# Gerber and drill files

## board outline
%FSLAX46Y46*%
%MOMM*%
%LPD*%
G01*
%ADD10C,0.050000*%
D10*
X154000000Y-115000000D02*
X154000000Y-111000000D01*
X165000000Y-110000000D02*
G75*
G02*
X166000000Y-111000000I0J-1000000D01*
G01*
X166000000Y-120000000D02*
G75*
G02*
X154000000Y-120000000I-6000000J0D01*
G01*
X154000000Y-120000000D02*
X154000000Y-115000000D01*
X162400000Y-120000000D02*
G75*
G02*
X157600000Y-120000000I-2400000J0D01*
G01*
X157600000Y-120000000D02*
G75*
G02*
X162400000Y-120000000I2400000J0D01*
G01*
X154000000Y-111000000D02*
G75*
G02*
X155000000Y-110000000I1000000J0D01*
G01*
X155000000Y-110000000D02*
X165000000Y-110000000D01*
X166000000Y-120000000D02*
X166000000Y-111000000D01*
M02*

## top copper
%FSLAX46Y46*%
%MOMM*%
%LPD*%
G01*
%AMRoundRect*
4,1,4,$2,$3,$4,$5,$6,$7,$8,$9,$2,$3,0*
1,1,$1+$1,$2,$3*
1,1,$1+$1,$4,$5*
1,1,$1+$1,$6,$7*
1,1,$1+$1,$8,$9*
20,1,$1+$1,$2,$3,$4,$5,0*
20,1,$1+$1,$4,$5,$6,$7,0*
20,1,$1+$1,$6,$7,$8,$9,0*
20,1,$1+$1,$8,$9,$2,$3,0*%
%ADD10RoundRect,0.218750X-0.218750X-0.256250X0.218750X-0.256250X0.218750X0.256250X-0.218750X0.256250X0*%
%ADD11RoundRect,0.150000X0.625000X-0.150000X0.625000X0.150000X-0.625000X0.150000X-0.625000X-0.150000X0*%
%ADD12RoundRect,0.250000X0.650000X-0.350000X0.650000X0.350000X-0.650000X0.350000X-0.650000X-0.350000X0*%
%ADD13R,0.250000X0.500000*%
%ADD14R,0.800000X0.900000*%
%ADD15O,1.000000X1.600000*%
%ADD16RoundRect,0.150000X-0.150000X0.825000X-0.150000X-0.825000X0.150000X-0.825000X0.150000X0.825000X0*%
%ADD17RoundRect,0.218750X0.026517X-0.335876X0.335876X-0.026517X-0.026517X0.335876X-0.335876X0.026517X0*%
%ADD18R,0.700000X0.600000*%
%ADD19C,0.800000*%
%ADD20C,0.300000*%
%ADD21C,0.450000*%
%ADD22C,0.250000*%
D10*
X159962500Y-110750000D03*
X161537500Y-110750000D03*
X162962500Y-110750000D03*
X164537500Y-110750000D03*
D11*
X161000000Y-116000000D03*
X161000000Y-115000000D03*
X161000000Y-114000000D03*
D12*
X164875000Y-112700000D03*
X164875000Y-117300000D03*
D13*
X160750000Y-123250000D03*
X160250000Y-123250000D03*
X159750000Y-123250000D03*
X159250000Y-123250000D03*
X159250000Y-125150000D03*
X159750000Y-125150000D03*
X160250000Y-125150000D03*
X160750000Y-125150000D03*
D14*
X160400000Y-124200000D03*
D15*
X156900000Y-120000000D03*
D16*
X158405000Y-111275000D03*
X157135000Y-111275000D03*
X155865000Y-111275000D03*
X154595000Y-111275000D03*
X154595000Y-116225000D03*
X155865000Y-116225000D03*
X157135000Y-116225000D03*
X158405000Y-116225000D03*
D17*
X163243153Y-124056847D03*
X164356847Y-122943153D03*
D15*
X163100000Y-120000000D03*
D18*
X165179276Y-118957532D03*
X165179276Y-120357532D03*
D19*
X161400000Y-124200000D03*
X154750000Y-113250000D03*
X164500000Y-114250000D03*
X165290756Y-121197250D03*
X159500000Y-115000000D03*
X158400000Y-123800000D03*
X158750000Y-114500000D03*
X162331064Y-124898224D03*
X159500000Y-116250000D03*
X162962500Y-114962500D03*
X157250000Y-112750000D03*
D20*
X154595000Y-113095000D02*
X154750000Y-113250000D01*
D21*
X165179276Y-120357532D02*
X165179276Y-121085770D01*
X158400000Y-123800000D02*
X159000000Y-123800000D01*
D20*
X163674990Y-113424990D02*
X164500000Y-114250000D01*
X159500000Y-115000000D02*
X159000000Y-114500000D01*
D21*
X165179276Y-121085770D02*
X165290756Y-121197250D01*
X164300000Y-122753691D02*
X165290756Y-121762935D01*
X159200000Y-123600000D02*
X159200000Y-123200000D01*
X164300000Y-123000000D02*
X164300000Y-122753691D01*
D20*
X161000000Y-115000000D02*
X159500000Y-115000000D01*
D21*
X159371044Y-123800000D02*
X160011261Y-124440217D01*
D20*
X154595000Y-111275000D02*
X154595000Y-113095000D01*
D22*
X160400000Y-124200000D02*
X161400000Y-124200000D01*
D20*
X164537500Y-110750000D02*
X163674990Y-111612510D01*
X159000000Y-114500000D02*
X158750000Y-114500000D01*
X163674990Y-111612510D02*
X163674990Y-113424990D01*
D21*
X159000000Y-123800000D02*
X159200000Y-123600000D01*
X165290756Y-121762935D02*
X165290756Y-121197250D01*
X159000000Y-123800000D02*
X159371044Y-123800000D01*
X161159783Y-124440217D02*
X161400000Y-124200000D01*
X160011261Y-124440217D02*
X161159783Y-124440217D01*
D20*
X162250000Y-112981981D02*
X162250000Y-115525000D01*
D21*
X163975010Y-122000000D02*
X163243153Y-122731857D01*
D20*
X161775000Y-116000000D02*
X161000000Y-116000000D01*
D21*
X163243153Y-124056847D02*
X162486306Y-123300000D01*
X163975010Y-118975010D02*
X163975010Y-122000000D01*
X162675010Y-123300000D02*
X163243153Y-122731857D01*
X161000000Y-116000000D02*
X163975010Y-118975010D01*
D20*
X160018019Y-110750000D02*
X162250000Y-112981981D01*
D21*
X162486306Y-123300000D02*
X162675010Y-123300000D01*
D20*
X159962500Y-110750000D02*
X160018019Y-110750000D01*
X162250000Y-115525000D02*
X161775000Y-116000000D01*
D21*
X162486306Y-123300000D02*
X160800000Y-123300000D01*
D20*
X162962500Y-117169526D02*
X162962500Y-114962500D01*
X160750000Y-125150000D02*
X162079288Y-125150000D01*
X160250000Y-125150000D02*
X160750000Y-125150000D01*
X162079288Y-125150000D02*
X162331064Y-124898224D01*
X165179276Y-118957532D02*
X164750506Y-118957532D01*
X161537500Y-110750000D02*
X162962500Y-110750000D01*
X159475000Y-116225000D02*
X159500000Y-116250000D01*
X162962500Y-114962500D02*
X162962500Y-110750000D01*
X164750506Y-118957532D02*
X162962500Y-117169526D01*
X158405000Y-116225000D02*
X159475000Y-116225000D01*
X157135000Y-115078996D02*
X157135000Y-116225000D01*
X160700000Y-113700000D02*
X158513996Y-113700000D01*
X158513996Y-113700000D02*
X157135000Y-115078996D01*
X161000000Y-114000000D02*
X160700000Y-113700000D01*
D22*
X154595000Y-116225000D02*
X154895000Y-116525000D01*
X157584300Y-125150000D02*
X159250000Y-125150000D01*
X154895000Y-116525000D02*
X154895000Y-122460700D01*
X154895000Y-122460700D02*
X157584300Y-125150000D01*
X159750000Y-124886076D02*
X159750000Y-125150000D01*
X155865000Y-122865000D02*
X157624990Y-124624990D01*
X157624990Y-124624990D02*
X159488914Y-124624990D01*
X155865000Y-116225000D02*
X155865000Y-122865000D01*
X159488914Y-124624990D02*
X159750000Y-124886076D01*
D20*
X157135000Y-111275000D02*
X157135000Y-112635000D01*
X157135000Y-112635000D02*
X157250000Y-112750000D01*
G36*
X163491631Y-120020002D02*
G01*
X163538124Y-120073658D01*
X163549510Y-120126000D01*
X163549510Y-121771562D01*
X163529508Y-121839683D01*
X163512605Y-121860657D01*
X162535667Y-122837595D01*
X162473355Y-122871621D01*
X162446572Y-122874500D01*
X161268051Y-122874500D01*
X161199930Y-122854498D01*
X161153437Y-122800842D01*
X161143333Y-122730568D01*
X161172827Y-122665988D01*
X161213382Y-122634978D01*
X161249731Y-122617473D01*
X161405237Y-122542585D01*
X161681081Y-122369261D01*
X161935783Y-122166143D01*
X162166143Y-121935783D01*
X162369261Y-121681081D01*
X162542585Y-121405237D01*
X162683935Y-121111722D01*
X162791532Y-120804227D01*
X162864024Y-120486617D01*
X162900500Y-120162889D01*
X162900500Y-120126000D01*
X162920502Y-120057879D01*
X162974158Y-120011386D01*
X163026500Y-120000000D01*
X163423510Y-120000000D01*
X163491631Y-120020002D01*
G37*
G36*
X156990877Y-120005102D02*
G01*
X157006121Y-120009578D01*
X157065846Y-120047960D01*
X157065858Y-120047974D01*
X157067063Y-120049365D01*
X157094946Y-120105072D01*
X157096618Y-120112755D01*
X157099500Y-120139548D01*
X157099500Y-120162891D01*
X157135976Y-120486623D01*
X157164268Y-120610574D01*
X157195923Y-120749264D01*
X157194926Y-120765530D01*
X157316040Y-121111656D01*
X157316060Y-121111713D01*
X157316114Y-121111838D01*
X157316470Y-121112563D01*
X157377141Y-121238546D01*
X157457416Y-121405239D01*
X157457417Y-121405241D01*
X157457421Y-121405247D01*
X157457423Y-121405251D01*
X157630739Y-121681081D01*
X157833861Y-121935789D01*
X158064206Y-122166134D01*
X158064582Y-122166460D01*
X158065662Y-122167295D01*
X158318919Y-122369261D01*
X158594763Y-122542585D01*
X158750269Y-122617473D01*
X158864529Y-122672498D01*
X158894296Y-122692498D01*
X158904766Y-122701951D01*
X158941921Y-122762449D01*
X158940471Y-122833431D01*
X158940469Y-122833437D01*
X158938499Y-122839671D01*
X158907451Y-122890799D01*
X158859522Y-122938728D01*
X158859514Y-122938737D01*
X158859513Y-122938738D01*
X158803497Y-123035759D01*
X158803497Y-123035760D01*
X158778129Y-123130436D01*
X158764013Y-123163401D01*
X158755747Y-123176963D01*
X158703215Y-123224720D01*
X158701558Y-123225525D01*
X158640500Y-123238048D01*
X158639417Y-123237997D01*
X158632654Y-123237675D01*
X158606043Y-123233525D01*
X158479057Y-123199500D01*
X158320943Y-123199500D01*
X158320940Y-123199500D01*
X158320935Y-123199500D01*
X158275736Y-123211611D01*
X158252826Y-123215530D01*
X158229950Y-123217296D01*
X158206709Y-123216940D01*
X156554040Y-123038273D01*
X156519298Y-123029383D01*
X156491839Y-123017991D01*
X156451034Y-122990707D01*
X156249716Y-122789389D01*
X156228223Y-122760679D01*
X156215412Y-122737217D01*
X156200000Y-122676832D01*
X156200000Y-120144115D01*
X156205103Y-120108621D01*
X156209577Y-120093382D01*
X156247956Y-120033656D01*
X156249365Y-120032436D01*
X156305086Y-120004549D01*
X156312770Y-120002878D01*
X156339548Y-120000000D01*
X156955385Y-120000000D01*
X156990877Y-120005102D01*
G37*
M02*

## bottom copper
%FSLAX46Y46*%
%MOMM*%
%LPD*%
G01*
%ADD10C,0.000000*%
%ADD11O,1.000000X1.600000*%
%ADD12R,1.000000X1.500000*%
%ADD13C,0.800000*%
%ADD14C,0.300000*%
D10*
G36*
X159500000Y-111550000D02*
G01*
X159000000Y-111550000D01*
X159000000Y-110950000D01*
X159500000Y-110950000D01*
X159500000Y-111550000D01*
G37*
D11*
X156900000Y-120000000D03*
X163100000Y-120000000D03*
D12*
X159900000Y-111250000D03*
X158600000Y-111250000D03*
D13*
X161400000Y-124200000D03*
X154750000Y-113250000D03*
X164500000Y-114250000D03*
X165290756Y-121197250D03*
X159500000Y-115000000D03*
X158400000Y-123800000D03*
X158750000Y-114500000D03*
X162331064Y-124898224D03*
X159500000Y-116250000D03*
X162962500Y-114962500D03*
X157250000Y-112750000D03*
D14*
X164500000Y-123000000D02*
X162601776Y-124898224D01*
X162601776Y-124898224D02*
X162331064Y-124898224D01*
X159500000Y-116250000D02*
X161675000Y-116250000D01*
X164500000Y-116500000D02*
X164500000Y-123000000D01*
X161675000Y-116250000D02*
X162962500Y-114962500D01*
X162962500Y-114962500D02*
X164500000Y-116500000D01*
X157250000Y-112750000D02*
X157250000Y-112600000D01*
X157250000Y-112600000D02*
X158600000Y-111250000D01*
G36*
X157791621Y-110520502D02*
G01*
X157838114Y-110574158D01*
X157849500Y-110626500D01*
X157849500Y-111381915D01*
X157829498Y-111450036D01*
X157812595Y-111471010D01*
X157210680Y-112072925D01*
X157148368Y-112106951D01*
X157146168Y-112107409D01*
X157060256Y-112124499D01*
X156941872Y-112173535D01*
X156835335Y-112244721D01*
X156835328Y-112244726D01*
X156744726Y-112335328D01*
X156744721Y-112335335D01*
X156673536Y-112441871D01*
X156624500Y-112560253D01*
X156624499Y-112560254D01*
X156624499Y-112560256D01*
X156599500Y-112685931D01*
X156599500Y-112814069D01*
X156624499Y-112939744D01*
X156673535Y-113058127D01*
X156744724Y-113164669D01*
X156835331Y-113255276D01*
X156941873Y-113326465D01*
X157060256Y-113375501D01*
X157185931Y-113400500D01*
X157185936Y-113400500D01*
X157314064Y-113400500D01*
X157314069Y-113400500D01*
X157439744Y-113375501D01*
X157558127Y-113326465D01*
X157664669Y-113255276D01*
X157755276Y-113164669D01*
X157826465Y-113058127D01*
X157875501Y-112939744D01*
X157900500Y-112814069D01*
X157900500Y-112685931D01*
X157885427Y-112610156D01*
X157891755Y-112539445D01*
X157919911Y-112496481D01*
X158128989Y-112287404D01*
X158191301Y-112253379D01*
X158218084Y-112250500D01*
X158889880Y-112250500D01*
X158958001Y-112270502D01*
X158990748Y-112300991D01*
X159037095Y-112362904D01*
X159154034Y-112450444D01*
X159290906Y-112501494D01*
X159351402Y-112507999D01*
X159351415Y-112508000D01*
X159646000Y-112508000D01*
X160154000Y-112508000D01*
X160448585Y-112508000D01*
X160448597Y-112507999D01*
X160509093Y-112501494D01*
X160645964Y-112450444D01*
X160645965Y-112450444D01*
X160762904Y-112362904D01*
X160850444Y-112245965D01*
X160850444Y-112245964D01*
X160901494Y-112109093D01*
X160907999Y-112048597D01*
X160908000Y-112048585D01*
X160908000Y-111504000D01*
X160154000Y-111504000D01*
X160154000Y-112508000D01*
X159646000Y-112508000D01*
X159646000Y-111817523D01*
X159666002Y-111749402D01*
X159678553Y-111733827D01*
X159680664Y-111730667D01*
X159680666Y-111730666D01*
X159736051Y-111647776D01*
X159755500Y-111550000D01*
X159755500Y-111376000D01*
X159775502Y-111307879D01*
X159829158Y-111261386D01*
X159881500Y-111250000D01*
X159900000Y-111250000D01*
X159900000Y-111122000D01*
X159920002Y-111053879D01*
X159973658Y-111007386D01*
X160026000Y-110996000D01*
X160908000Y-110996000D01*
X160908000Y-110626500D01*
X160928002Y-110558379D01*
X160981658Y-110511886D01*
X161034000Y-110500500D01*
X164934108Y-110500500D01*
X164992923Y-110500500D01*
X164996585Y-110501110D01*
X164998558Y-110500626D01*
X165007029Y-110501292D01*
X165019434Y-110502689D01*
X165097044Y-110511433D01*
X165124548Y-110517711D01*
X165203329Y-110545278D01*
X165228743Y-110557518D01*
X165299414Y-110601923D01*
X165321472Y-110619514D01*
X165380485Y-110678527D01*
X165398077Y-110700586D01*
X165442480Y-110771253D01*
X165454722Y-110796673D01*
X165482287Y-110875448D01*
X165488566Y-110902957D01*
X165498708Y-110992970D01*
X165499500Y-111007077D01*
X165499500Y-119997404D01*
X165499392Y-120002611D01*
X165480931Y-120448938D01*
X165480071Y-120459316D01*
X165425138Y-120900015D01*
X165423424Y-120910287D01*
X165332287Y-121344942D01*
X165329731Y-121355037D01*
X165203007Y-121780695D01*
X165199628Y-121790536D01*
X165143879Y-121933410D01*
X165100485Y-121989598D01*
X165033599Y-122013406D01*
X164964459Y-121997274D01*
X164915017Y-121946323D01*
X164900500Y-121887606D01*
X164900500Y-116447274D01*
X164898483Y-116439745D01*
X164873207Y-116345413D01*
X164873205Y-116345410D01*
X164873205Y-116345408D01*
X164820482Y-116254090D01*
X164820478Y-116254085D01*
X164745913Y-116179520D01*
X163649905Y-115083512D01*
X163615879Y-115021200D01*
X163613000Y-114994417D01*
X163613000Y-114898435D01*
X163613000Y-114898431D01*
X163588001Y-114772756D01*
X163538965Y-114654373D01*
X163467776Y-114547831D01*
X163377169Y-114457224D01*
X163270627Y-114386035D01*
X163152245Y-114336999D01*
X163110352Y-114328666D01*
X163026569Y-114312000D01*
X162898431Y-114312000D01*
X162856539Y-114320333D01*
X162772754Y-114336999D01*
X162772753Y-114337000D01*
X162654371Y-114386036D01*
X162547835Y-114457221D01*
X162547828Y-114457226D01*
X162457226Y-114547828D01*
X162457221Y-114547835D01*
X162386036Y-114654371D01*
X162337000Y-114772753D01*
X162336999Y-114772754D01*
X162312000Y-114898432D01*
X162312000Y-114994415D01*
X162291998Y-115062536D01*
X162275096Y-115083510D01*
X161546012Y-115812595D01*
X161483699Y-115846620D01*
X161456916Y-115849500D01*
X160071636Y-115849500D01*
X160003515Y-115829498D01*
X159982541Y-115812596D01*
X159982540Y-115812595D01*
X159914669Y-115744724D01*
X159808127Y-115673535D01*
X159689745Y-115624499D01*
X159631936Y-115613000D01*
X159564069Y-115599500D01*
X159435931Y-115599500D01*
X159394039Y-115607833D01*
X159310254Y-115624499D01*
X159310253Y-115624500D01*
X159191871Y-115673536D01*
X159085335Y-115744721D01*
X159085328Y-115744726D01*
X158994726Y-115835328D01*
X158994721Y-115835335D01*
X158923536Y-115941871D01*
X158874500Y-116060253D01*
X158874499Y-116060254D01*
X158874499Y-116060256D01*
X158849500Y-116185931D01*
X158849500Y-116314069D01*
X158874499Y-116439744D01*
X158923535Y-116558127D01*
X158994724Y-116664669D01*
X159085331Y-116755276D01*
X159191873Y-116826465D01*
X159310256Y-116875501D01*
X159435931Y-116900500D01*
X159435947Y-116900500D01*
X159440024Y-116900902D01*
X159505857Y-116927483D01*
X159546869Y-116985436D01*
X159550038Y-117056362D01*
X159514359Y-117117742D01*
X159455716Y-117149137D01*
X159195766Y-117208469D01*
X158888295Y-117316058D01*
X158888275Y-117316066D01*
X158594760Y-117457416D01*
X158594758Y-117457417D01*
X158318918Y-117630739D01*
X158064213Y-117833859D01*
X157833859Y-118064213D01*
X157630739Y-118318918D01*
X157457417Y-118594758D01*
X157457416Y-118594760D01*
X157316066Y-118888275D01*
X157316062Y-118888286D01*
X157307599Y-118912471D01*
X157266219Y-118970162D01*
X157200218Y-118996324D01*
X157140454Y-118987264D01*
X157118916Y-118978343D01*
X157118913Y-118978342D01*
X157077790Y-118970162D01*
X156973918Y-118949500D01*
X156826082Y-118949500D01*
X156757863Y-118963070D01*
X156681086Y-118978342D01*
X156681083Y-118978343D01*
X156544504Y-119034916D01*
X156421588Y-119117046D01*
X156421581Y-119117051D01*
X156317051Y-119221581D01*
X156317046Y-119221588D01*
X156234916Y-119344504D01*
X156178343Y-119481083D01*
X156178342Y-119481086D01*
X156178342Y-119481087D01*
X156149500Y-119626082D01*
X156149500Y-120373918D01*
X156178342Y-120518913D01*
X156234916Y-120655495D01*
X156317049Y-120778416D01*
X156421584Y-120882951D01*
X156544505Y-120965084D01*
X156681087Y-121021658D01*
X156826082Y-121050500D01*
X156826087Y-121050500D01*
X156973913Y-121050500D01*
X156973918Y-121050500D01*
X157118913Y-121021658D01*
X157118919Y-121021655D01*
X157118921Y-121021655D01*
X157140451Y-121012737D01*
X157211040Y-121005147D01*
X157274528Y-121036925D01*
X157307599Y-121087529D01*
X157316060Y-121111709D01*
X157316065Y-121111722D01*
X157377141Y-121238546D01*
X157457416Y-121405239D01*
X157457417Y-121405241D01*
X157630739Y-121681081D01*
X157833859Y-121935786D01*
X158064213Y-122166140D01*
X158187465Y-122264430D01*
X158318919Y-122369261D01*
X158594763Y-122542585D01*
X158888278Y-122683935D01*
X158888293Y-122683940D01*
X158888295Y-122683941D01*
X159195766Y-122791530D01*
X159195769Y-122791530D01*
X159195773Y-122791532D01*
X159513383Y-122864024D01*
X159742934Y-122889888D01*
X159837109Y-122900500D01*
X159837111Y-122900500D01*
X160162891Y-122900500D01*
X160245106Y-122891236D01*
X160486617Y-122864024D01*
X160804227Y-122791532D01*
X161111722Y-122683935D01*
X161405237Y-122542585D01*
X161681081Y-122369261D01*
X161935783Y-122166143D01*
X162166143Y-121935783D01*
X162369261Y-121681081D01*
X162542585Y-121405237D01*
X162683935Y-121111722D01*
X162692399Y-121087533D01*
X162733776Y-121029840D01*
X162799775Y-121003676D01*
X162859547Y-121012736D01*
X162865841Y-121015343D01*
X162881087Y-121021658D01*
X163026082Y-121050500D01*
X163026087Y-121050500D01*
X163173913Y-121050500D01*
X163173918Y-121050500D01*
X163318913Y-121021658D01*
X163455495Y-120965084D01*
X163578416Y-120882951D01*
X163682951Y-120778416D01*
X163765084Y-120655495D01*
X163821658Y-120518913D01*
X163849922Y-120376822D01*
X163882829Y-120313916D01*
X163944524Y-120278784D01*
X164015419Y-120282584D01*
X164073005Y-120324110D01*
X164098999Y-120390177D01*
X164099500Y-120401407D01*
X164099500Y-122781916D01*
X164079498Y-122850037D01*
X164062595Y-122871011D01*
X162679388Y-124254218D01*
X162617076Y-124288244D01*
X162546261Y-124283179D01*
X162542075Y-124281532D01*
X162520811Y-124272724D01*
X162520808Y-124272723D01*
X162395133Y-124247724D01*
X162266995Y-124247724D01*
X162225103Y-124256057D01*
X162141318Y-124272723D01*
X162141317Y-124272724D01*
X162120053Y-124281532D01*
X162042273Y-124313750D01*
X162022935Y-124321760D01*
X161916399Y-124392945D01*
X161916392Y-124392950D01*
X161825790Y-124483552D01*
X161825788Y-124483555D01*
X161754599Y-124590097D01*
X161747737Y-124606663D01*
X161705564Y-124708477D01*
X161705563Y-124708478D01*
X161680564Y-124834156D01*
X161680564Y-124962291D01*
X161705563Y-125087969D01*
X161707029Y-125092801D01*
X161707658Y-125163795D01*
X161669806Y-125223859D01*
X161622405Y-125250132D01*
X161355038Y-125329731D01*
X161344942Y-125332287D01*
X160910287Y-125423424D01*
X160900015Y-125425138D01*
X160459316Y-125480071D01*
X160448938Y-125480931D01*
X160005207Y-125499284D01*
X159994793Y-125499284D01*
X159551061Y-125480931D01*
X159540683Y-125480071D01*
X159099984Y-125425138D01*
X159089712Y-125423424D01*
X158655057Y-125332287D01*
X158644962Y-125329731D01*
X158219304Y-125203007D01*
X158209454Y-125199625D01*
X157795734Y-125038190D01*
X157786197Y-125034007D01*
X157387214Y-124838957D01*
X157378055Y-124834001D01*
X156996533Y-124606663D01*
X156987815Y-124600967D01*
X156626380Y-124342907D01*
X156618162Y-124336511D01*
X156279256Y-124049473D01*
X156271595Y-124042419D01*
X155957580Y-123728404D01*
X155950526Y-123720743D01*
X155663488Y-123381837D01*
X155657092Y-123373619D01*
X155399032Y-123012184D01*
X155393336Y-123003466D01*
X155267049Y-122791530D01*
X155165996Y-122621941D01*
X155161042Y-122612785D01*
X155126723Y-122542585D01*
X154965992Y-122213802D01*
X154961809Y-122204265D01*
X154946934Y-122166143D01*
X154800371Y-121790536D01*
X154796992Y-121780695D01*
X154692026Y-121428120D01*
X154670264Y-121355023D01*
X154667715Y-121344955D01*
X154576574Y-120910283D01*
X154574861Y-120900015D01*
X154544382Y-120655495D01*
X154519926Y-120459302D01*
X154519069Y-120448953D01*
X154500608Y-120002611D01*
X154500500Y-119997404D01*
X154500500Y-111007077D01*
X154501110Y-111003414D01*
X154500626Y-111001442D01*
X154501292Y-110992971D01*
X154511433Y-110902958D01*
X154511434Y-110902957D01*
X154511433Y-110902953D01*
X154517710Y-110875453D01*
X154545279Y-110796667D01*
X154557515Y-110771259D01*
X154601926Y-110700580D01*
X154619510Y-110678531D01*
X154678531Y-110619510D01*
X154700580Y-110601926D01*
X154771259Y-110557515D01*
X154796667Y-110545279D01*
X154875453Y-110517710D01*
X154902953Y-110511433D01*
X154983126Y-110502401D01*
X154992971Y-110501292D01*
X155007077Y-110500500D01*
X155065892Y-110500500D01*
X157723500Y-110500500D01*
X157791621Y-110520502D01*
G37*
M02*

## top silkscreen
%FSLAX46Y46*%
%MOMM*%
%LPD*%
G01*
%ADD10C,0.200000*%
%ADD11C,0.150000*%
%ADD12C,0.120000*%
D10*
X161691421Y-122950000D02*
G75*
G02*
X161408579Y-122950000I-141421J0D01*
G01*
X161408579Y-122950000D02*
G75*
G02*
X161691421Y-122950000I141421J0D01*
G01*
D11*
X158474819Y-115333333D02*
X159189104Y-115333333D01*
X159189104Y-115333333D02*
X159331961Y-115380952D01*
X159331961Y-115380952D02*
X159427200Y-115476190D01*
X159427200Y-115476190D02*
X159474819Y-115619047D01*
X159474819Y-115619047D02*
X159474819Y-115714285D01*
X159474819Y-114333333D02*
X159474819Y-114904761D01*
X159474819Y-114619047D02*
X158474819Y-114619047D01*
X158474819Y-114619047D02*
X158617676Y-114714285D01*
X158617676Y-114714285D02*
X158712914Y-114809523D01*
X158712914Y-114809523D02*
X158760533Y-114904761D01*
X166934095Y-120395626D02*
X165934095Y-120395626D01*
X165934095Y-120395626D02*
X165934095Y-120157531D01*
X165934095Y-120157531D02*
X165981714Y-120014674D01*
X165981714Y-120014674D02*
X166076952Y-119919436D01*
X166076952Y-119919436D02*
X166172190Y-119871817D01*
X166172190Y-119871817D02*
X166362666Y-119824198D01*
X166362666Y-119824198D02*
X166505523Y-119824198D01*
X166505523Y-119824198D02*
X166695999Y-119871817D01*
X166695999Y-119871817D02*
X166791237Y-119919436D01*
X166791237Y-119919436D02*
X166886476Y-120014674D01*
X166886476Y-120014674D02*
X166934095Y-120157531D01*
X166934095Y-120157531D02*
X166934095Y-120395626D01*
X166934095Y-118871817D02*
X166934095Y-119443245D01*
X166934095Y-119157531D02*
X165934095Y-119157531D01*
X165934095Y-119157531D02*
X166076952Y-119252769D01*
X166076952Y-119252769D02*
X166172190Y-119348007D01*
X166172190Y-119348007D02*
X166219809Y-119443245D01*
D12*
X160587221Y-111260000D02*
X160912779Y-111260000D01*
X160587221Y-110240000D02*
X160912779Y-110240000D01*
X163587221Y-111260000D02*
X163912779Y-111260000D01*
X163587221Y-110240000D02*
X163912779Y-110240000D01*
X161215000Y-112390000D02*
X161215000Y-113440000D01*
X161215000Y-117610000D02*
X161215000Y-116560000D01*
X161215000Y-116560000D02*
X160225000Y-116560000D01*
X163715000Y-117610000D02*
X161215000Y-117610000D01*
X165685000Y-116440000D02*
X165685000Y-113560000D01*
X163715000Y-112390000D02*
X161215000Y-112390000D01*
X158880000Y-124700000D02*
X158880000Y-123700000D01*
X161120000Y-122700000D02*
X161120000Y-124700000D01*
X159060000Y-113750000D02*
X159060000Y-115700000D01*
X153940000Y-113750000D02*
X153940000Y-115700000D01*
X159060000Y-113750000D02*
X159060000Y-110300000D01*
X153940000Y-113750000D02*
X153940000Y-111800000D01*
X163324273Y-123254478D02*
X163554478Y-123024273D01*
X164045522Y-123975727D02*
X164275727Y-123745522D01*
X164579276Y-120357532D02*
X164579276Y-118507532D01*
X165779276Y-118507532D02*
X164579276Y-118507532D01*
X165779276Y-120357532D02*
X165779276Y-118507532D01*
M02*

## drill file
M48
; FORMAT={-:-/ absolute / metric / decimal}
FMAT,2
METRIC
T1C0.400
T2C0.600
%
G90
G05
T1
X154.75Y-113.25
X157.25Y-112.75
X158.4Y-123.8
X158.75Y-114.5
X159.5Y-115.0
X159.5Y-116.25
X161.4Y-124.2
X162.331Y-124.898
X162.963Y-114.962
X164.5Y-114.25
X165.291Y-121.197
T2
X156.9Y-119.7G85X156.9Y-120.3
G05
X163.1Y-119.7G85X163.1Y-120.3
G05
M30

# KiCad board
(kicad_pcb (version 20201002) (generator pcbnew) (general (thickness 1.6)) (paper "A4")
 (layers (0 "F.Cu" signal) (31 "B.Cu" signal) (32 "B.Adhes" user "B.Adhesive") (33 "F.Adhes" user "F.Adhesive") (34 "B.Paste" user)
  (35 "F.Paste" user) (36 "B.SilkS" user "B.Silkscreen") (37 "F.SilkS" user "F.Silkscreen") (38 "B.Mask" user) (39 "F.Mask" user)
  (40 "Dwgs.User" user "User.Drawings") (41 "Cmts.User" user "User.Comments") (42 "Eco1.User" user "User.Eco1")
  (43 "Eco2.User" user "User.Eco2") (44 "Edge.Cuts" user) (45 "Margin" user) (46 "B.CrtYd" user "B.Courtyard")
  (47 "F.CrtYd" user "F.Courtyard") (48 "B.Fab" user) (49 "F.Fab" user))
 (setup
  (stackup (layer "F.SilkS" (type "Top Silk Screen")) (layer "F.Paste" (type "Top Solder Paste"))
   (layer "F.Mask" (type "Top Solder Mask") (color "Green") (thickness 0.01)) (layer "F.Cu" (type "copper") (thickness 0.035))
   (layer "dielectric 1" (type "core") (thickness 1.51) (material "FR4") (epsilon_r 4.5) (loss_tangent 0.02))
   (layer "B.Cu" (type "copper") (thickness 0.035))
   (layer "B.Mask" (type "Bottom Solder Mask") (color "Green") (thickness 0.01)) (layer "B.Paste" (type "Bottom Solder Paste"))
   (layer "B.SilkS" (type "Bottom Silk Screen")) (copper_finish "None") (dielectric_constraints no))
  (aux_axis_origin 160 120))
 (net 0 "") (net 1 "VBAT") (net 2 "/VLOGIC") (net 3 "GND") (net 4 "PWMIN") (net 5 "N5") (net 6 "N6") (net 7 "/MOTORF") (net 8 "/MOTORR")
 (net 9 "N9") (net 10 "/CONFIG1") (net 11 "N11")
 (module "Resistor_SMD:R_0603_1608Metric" (layer "F.Cu") (at 160.75 110.75)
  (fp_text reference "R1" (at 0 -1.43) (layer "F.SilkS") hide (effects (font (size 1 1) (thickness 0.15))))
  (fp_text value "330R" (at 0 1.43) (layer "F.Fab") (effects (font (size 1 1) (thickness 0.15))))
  (fp_line (start -0.162779 0.51) (end 0.162779 0.51) (layer "F.SilkS") (width 0.12))
  (fp_line (start -0.162779 -0.51) (end 0.162779 -0.51) (layer "F.SilkS") (width 0.12))
  (pad "1" smd roundrect (at -0.7875 0) (size 0.875 0.95) (layers "F.Cu" "F.Paste" "F.Mask") (roundrect_rratio 0.25) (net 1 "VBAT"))
  (pad "2" smd roundrect (at 0.7875 0) (size 0.875 0.95) (layers "F.Cu" "F.Paste" "F.Mask") (roundrect_rratio 0.25) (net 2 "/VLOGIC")))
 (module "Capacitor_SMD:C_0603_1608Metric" (layer "F.Cu") (at 163.75 110.75)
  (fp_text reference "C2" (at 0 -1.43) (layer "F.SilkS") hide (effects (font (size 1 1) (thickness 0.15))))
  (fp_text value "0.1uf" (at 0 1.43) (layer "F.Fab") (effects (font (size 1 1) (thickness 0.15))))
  (fp_line (start -0.162779 0.51) (end 0.162779 0.51) (layer "F.SilkS") (width 0.12))
  (fp_line (start -0.162779 -0.51) (end 0.162779 -0.51) (layer "F.SilkS") (width 0.12))
  (pad "1" smd roundrect (at -0.7875 0) (size 0.875 0.95) (layers "F.Cu" "F.Paste" "F.Mask") (roundrect_rratio 0.25) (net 2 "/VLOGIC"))
  (pad "2" smd roundrect (at 0.7875 0) (size 0.875 0.95) (layers "F.Cu" "F.Paste" "F.Mask") (roundrect_rratio 0.25) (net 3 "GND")))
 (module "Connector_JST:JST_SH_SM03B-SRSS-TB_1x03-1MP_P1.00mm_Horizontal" (layer "F.Cu") (at 163 115 90)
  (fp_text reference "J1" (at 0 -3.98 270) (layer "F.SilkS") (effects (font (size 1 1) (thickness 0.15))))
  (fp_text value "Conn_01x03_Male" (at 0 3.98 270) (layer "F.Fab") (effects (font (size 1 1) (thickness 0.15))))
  (fp_line (start 2.61 -1.785) (end 1.56 -1.785) (layer "F.SilkS") (width 0.12))
  (fp_line (start -2.61 -1.785) (end -1.56 -1.785) (layer "F.SilkS") (width 0.12))
  (fp_line (start -1.56 -1.785) (end -1.56 -2.775) (layer "F.SilkS") (width 0.12))
  (fp_line (start -2.61 0.715) (end -2.61 -1.785) (layer "F.SilkS") (width 0.12))
  (fp_line (start -1.44 2.685) (end 1.44 2.685) (layer "F.SilkS") (width 0.12))
  (fp_line (start 2.61 0.715) (end 2.61 -1.785) (layer "F.SilkS") (width 0.12))
  (pad "1" smd roundrect (at -1 -2 90) (size 0.6 1.55) (layers "F.Cu" "F.Paste" "F.Mask") (roundrect_rratio 0.25) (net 1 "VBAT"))
  (pad "2" smd roundrect (at 0 -2 90) (size 0.6 1.55) (layers "F.Cu" "F.Paste" "F.Mask") (roundrect_rratio 0.25) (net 3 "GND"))
  (pad "3" smd roundrect (at 1 -2 90) (size 0.6 1.55) (layers "F.Cu" "F.Paste" "F.Mask") (roundrect_rratio 0.25) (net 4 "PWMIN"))
  (pad "MP" smd roundrect (at 2.3 1.875 90) (size 1.2 1.8) (layers "F.Cu" "F.Paste" "F.Mask") (roundrect_rratio 0.208333))
  (pad "MP" smd roundrect (at -2.3 1.875 90) (size 1.2 1.8) (layers "F.Cu" "F.Paste" "F.Mask") (roundrect_rratio 0.208333)))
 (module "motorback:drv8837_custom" (layer "F.Cu") (at 160 124.2 -90)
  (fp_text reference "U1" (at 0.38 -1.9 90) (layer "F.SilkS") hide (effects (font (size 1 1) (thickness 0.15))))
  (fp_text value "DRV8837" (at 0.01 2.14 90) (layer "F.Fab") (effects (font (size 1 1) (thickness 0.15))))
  (fp_line (start 0.5 1.12) (end -0.5 1.12) (layer "F.SilkS") (width 0.12))
  (fp_line (start -1.5 -1.12) (end 0.5 -1.12) (layer "F.SilkS") (width 0.12))
  (pad "" smd rect (at 0 -0.4 270) (size 0.75 0.65) (layers "F.Paste"))
  (pad "1" smd rect (at -0.95 -0.75 270) (size 0.5 0.25) (layers "F.Cu" "F.Paste" "F.Mask") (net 1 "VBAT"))
  (pad "2" smd rect (at -0.95 -0.25 270) (size 0.5 0.25) (layers "F.Cu" "F.Paste" "F.Mask") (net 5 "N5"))
  (pad "3" smd rect (at -0.95 0.25 270) (size 0.5 0.25) (layers "F.Cu" "F.Paste" "F.Mask") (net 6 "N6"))
  (pad "4" smd rect (at -0.95 0.75 270) (size 0.5 0.25) (layers "F.Cu" "F.Paste" "F.Mask") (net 3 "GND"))
  (pad "5" smd rect (at 0.95 0.75 270) (size 0.5 0.25) (layers "F.Cu" "F.Paste" "F.Mask") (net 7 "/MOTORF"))
  (pad "6" smd rect (at 0.95 0.25 270) (size 0.5 0.25) (layers "F.Cu" "F.Paste" "F.Mask") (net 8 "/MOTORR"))
  (pad "7" smd rect (at 0.95 -0.25 270) (size 0.5 0.25) (layers "F.Cu" "F.Paste" "F.Mask") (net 2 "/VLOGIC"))
  (pad "8" smd rect (at 0.95 -0.75 270) (size 0.5 0.25) (layers "F.Cu" "F.Paste" "F.Mask") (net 2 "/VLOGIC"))
  (pad "9" smd rect (at 0 -0.4 270) (size 0.9 0.8) (layers "F.Cu" "F.Mask") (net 3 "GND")))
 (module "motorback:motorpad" (layer "F.Cu") (at 156.9 120)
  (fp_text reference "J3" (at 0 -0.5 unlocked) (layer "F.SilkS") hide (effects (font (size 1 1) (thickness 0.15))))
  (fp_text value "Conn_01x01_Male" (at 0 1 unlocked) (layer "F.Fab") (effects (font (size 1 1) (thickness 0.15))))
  (pad "1" thru_hole oval (at 0 0) (size 1 1.6) (drill oval 0.6 1.2) (layers *.Cu *.Mask) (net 6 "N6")))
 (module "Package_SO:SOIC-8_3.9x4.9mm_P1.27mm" (layer "F.Cu") (at 156.5 113.75 -90)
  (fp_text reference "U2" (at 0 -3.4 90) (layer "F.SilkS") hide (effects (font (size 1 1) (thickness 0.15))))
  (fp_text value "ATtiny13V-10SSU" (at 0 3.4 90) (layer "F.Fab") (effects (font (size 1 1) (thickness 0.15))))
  (fp_line (start 0 -2.56) (end 1.95 -2.56) (layer "F.SilkS") (width 0.12))
  (fp_line (start 0 2.56) (end 1.95 2.56) (layer "F.SilkS") (width 0.12))
  (fp_line (start 0 -2.56) (end -3.45 -2.56) (layer "F.SilkS") (width 0.12))
  (fp_line (start 0 2.56) (end -1.95 2.56) (layer "F.SilkS") (width 0.12))
  (pad "1" smd roundrect (at -2.475 -1.905 270) (size 1.95 0.6) (layers "F.Cu" "F.Paste" "F.Mask") (roundrect_rratio 0.25) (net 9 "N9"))
  (pad "2" smd roundrect (at -2.475 -0.635 270) (size 1.95 0.6) (layers "F.Cu" "F.Paste" "F.Mask") (roundrect_rratio 0.25)
   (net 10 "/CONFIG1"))
  (pad "3" smd roundrect (at -2.475 0.635 270) (size 1.95 0.6) (layers "F.Cu" "F.Paste" "F.Mask") (roundrect_rratio 0.25) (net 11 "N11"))
  (pad "4" smd roundrect (at -2.475 1.905 270) (size 1.95 0.6) (layers "F.Cu" "F.Paste" "F.Mask") (roundrect_rratio 0.25) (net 3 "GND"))
  (pad "5" smd roundrect (at 2.475 1.905 270) (size 1.95 0.6) (layers "F.Cu" "F.Paste" "F.Mask") (roundrect_rratio 0.25) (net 7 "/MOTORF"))
  (pad "6" smd roundrect (at 2.475 0.635 270) (size 1.95 0.6) (layers "F.Cu" "F.Paste" "F.Mask") (roundrect_rratio 0.25) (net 8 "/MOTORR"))
  (pad "7" smd roundrect (at 2.475 -0.635 270) (size 1.95 0.6) (layers "F.Cu" "F.Paste" "F.Mask") (roundrect_rratio 0.25) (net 4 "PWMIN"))
  (pad "8" smd roundrect (at 2.475 -1.905 270) (size 1.95 0.6) (layers "F.Cu" "F.Paste" "F.Mask") (roundrect_rratio 0.25) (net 2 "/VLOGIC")))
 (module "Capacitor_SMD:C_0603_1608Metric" (layer "F.Cu") (at 163.8 123.5 45)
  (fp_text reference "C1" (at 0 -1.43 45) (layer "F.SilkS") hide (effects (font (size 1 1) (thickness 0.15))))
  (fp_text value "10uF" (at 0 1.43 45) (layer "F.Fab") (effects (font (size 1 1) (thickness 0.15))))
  (fp_line (start -0.162779 -0.51) (end 0.162779 -0.51) (layer "F.SilkS") (width 0.12))
  (fp_line (start -0.162779 0.51) (end 0.162779 0.51) (layer "F.SilkS") (width 0.12))
  (pad "1" smd roundrect (at -0.7875 0 45) (size 0.875 0.95) (layers "F.Cu" "F.Paste" "F.Mask") (roundrect_rratio 0.25) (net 1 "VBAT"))
  (pad "2" smd roundrect (at 0.7875 0 45) (size 0.875 0.95) (layers "F.Cu" "F.Paste" "F.Mask") (roundrect_rratio 0.25) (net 3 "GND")))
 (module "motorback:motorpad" (layer "F.Cu") (at 163 120)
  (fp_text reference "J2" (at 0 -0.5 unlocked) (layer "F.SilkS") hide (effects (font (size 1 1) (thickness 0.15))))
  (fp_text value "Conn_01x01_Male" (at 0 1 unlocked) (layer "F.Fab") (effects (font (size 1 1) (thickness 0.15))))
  (pad "1" thru_hole oval (at 0.1 0) (size 1 1.6) (drill oval 0.6 1.2) (layers *.Cu *.Mask) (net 5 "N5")))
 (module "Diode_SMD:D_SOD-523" (layer "F.Cu") (at 165.179276 119.657532 -90)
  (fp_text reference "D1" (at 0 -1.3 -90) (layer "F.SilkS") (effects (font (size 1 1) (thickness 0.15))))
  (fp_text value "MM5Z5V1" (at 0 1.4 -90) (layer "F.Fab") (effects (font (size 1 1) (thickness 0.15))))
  (fp_line (start 0.7 0.6) (end -1.15 0.6) (layer "F.SilkS") (width 0.12))
  (fp_line (start -1.15 -0.6) (end -1.15 0.6) (layer "F.SilkS") (width 0.12))
  (fp_line (start 0.7 -0.6) (end -1.15 -0.6) (layer "F.SilkS") (width 0.12))
  (pad "1" smd rect (at -0.7 0 90) (size 0.6 0.7) (layers "F.Cu" "F.Paste" "F.Mask") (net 2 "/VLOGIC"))
  (pad "2" smd rect (at 0.7 0 90) (size 0.6 0.7) (layers "F.Cu" "F.Paste" "F.Mask") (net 3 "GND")))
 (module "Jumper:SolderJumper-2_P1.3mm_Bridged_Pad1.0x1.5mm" (layer "B.Cu") (at 159.25 111.25 180)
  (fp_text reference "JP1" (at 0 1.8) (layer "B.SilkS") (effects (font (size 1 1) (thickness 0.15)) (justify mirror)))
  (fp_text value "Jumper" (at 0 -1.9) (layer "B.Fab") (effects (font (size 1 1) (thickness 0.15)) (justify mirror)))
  (fp_poly (pts (xy -0.25 0.3) (xy 0.25 0.3) (xy 0.25 -0.3) (xy -0.25 -0.3)) (layer "B.Cu") (width 0))
  (pad "1" smd rect (at -0.65 0 180) (size 1 1.5) (layers "B.Cu" "B.Mask") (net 3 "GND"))
  (pad "2" smd rect (at 0.65 0 180) (size 1 1.5) (layers "B.Cu" "B.Mask") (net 10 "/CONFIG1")))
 (gr_circle (center 161.55 122.95) (end 161.691421 122.95) (layer "F.SilkS") (width 0.2))
 (gr_line (start 154 115) (end 154 111) (layer "Edge.Cuts") (width 0.05))
 (gr_arc (start 165 111) (end 166 111) (angle -90) (layer "Edge.Cuts") (width 0.05))
 (gr_arc (start 160 120) (end 154 120) (angle -180) (layer "Edge.Cuts") (width 0.05))
 (gr_line (start 154 120) (end 154 115) (layer "Edge.Cuts") (width 0.05))
 (gr_circle (center 160 120) (end 162.4 120) (layer "Edge.Cuts") (width 0.05))
 (gr_arc (start 155 111) (end 155 110) (angle -90) (layer "Edge.Cuts") (width 0.05))
 (gr_line (start 155 110) (end 165 110) (layer "Edge.Cuts") (width 0.05))
 (gr_line (start 166 120) (end 166 111) (layer "Edge.Cuts") (width 0.05))
 (segment (start 154.595 113.095) (end 154.75 113.25) (width 0.3) (layer "F.Cu") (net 3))
 (segment (start 165.179276 120.357532) (end 165.179276 121.08577) (width 0.45) (layer "F.Cu") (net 3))
 (segment (start 158.4 123.8) (end 159 123.8) (width 0.45) (layer "F.Cu") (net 3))
 (segment (start 163.67499 113.42499) (end 164.5 114.25) (width 0.3) (layer "F.Cu") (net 3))
 (segment (start 159.5 115) (end 159 114.5) (width 0.3) (layer "F.Cu") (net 3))
 (segment (start 165.179276 121.08577) (end 165.290756 121.19725) (width 0.45) (layer "F.Cu") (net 3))
 (segment (start 164.3 122.753691) (end 165.290756 121.762935) (width 0.45) (layer "F.Cu") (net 3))
 (segment (start 159.2 123.6) (end 159.2 123.2) (width 0.45) (layer "F.Cu") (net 3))
 (segment (start 164.3 123) (end 164.3 122.753691) (width 0.45) (layer "F.Cu") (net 3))
 (segment (start 161 115) (end 159.5 115) (width 0.3) (layer "F.Cu") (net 3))
 (segment (start 159.371044 123.8) (end 160.011261 124.440217) (width 0.45) (layer "F.Cu") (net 3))
 (segment (start 154.595 111.275) (end 154.595 113.095) (width 0.3) (layer "F.Cu") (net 3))
 (segment (start 160.4 124.2) (end 161.4 124.2) (width 0.25) (layer "F.Cu") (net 3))
 (segment (start 164.5375 110.75) (end 163.67499 111.61251) (width 0.3) (layer "F.Cu") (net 3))
 (segment (start 159 114.5) (end 158.75 114.5) (width 0.3) (layer "F.Cu") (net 3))
 (segment (start 163.67499 111.61251) (end 163.67499 113.42499) (width 0.3) (layer "F.Cu") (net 3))
 (segment (start 159 123.8) (end 159.2 123.6) (width 0.45) (layer "F.Cu") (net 3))
 (segment (start 165.290756 121.762935) (end 165.290756 121.19725) (width 0.45) (layer "F.Cu") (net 3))
 (segment (start 159 123.8) (end 159.371044 123.8) (width 0.45) (layer "F.Cu") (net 3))
 (segment (start 161.159783 124.440217) (end 161.4 124.2) (width 0.45) (layer "F.Cu") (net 3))
 (segment (start 160.011261 124.440217) (end 161.159783 124.440217) (width 0.45) (layer "F.Cu") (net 3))
 (via (at 161.4 124.2) (size 0.8) (drill 0.4) (layers "F.Cu" "B.Cu") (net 3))
 (via (at 154.75 113.25) (size 0.8) (drill 0.4) (layers "F.Cu" "B.Cu") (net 3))
 (via (at 164.5 114.25) (size 0.8) (drill 0.4) (layers "F.Cu" "B.Cu") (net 3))
 (via (at 165.290756 121.19725) (size 0.8) (drill 0.4) (layers "F.Cu" "B.Cu") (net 3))
 (via (at 159.5 115) (size 0.8) (drill 0.4) (layers "F.Cu" "B.Cu") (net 3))
 (via (at 158.4 123.8) (size 0.8) (drill 0.4) (layers "F.Cu" "B.Cu") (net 3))
 (via (at 158.75 114.5) (size 0.8) (drill 0.4) (layers "F.Cu" "B.Cu") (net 3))
 (segment (start 162.25 112.981981) (end 162.25 115.525) (width 0.3) (layer "F.Cu") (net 1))
 (segment (start 163.97501 122) (end 163.243153 122.731857) (width 0.45) (layer "F.Cu") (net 1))
 (segment (start 161.775 116) (end 161 116) (width 0.3) (layer "F.Cu") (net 1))
 (segment (start 163.243153 124.056847) (end 162.486306 123.3) (width 0.45) (layer "F.Cu") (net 1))
 (segment (start 163.97501 118.97501) (end 163.97501 122) (width 0.45) (layer "F.Cu") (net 1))
 (segment (start 162.67501 123.3) (end 163.243153 122.731857) (width 0.45) (layer "F.Cu") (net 1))
 (segment (start 161 116) (end 163.97501 118.97501) (width 0.45) (layer "F.Cu") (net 1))
 (segment (start 160.018019 110.75) (end 162.25 112.981981) (width 0.3) (layer "F.Cu") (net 1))
 (segment (start 162.486306 123.3) (end 162.67501 123.3) (width 0.45) (layer "F.Cu") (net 1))
 (segment (start 159.9625 110.75) (end 160.018019 110.75) (width 0.3) (layer "F.Cu") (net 1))
 (segment (start 162.25 115.525) (end 161.775 116) (width 0.3) (layer "F.Cu") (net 1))
 (segment (start 162.486306 123.3) (end 160.8 123.3) (width 0.45) (layer "F.Cu") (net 1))
 (segment (start 162.9625 117.169526) (end 162.9625 114.9625) (width 0.3) (layer "F.Cu") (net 2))
 (segment (start 160.75 125.15) (end 162.079288 125.15) (width 0.3) (layer "F.Cu") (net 2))
 (segment (start 160.25 125.15) (end 160.75 125.15) (width 0.3) (layer "F.Cu") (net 2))
 (segment (start 162.079288 125.15) (end 162.331064 124.898224) (width 0.3) (layer "F.Cu") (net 2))
 (segment (start 165.179276 118.957532) (end 164.750506 118.957532) (width 0.3) (layer "F.Cu") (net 2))
 (segment (start 161.5375 110.75) (end 162.9625 110.75) (width 0.3) (layer "F.Cu") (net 2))
 (segment (start 159.475 116.225) (end 159.5 116.25) (width 0.3) (layer "F.Cu") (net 2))
 (segment (start 162.9625 114.9625) (end 162.9625 110.75) (width 0.3) (layer "F.Cu") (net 2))
 (segment (start 164.750506 118.957532) (end 162.9625 117.169526) (width 0.3) (layer "F.Cu") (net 2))
 (segment (start 158.405 116.225) (end 159.475 116.225) (width 0.3) (layer "F.Cu") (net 2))
 (via (at 162.331064 124.898224) (size 0.8) (drill 0.4) (layers "F.Cu" "B.Cu") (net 2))
 (via (at 159.5 116.25) (size 0.8) (drill 0.4) (layers "F.Cu" "B.Cu") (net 2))
 (via (at 162.9625 114.9625) (size 0.8) (drill 0.4) (layers "F.Cu" "B.Cu") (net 2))
 (segment (start 164.5 123) (end 162.601776 124.898224) (width 0.3) (layer "B.Cu") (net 2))
 (segment (start 162.601776 124.898224) (end 162.331064 124.898224) (width 0.3) (layer "B.Cu") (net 2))
 (segment (start 159.5 116.25) (end 161.675 116.25) (width 0.3) (layer "B.Cu") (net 2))
 (segment (start 164.5 116.5) (end 164.5 123) (width 0.3) (layer "B.Cu") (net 2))
 (segment (start 161.675 116.25) (end 162.9625 114.9625) (width 0.3) (layer "B.Cu") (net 2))
 (segment (start 162.9625 114.9625) (end 164.5 116.5) (width 0.3) (layer "B.Cu") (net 2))
 (segment (start 157.135 115.078996) (end 157.135 116.225) (width 0.3) (layer "F.Cu") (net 4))
 (segment (start 160.7 113.7) (end 158.513996 113.7) (width 0.3) (layer "F.Cu") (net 4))
 (segment (start 158.513996 113.7) (end 157.135 115.078996) (width 0.3) (layer "F.Cu") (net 4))
 (segment (start 161 114) (end 160.7 113.7) (width 0.3) (layer "F.Cu") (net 4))
 (segment (start 154.595 116.225) (end 154.895 116.525) (width 0.25) (layer "F.Cu") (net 7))
 (segment (start 157.5843 125.15) (end 159.25 125.15) (width 0.25) (layer "F.Cu") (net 7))
 (segment (start 154.895 116.525) (end 154.895 122.4607) (width 0.25) (layer "F.Cu") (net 7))
 (segment (start 154.895 122.4607) (end 157.5843 125.15) (width 0.25) (layer "F.Cu") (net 7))
 (segment (start 159.75 124.886076) (end 159.75 125.15) (width 0.25) (layer "F.Cu") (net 8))
 (segment (start 155.865 122.865) (end 157.62499 124.62499) (width 0.25) (layer "F.Cu") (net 8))
 (segment (start 157.62499 124.62499) (end 159.488914 124.62499) (width 0.25) (layer "F.Cu") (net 8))
 (segment (start 155.865 116.225) (end 155.865 122.865) (width 0.25) (layer "F.Cu") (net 8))
 (segment (start 159.488914 124.62499) (end 159.75 124.886076) (width 0.25) (layer "F.Cu") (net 8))
 (segment (start 157.135 111.275) (end 157.135 112.635) (width 0.3) (layer "F.Cu") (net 10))
 (segment (start 157.135 112.635) (end 157.25 112.75) (width 0.3) (layer "F.Cu") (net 10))
 (via (at 157.25 112.75) (size 0.8) (drill 0.4) (layers "F.Cu" "B.Cu") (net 10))
 (segment (start 157.25 112.75) (end 157.25 112.6) (width 0.3) (layer "B.Cu") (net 10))
 (segment (start 157.25 112.6) (end 158.6 111.25) (width 0.3) (layer "B.Cu") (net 10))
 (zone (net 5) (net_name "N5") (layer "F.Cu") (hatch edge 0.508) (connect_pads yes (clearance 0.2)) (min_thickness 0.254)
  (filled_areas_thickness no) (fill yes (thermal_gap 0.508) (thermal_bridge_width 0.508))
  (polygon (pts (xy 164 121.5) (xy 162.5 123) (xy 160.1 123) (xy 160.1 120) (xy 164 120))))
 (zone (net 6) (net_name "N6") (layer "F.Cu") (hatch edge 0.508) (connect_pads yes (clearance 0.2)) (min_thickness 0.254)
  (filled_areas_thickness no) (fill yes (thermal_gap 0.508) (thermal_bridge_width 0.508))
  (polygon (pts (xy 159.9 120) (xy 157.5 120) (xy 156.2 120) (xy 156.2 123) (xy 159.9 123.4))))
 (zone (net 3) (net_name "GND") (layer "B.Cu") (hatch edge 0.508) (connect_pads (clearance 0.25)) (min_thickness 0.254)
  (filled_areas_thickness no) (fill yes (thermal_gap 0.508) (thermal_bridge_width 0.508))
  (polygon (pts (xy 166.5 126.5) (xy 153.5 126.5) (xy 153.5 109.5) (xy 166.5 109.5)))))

